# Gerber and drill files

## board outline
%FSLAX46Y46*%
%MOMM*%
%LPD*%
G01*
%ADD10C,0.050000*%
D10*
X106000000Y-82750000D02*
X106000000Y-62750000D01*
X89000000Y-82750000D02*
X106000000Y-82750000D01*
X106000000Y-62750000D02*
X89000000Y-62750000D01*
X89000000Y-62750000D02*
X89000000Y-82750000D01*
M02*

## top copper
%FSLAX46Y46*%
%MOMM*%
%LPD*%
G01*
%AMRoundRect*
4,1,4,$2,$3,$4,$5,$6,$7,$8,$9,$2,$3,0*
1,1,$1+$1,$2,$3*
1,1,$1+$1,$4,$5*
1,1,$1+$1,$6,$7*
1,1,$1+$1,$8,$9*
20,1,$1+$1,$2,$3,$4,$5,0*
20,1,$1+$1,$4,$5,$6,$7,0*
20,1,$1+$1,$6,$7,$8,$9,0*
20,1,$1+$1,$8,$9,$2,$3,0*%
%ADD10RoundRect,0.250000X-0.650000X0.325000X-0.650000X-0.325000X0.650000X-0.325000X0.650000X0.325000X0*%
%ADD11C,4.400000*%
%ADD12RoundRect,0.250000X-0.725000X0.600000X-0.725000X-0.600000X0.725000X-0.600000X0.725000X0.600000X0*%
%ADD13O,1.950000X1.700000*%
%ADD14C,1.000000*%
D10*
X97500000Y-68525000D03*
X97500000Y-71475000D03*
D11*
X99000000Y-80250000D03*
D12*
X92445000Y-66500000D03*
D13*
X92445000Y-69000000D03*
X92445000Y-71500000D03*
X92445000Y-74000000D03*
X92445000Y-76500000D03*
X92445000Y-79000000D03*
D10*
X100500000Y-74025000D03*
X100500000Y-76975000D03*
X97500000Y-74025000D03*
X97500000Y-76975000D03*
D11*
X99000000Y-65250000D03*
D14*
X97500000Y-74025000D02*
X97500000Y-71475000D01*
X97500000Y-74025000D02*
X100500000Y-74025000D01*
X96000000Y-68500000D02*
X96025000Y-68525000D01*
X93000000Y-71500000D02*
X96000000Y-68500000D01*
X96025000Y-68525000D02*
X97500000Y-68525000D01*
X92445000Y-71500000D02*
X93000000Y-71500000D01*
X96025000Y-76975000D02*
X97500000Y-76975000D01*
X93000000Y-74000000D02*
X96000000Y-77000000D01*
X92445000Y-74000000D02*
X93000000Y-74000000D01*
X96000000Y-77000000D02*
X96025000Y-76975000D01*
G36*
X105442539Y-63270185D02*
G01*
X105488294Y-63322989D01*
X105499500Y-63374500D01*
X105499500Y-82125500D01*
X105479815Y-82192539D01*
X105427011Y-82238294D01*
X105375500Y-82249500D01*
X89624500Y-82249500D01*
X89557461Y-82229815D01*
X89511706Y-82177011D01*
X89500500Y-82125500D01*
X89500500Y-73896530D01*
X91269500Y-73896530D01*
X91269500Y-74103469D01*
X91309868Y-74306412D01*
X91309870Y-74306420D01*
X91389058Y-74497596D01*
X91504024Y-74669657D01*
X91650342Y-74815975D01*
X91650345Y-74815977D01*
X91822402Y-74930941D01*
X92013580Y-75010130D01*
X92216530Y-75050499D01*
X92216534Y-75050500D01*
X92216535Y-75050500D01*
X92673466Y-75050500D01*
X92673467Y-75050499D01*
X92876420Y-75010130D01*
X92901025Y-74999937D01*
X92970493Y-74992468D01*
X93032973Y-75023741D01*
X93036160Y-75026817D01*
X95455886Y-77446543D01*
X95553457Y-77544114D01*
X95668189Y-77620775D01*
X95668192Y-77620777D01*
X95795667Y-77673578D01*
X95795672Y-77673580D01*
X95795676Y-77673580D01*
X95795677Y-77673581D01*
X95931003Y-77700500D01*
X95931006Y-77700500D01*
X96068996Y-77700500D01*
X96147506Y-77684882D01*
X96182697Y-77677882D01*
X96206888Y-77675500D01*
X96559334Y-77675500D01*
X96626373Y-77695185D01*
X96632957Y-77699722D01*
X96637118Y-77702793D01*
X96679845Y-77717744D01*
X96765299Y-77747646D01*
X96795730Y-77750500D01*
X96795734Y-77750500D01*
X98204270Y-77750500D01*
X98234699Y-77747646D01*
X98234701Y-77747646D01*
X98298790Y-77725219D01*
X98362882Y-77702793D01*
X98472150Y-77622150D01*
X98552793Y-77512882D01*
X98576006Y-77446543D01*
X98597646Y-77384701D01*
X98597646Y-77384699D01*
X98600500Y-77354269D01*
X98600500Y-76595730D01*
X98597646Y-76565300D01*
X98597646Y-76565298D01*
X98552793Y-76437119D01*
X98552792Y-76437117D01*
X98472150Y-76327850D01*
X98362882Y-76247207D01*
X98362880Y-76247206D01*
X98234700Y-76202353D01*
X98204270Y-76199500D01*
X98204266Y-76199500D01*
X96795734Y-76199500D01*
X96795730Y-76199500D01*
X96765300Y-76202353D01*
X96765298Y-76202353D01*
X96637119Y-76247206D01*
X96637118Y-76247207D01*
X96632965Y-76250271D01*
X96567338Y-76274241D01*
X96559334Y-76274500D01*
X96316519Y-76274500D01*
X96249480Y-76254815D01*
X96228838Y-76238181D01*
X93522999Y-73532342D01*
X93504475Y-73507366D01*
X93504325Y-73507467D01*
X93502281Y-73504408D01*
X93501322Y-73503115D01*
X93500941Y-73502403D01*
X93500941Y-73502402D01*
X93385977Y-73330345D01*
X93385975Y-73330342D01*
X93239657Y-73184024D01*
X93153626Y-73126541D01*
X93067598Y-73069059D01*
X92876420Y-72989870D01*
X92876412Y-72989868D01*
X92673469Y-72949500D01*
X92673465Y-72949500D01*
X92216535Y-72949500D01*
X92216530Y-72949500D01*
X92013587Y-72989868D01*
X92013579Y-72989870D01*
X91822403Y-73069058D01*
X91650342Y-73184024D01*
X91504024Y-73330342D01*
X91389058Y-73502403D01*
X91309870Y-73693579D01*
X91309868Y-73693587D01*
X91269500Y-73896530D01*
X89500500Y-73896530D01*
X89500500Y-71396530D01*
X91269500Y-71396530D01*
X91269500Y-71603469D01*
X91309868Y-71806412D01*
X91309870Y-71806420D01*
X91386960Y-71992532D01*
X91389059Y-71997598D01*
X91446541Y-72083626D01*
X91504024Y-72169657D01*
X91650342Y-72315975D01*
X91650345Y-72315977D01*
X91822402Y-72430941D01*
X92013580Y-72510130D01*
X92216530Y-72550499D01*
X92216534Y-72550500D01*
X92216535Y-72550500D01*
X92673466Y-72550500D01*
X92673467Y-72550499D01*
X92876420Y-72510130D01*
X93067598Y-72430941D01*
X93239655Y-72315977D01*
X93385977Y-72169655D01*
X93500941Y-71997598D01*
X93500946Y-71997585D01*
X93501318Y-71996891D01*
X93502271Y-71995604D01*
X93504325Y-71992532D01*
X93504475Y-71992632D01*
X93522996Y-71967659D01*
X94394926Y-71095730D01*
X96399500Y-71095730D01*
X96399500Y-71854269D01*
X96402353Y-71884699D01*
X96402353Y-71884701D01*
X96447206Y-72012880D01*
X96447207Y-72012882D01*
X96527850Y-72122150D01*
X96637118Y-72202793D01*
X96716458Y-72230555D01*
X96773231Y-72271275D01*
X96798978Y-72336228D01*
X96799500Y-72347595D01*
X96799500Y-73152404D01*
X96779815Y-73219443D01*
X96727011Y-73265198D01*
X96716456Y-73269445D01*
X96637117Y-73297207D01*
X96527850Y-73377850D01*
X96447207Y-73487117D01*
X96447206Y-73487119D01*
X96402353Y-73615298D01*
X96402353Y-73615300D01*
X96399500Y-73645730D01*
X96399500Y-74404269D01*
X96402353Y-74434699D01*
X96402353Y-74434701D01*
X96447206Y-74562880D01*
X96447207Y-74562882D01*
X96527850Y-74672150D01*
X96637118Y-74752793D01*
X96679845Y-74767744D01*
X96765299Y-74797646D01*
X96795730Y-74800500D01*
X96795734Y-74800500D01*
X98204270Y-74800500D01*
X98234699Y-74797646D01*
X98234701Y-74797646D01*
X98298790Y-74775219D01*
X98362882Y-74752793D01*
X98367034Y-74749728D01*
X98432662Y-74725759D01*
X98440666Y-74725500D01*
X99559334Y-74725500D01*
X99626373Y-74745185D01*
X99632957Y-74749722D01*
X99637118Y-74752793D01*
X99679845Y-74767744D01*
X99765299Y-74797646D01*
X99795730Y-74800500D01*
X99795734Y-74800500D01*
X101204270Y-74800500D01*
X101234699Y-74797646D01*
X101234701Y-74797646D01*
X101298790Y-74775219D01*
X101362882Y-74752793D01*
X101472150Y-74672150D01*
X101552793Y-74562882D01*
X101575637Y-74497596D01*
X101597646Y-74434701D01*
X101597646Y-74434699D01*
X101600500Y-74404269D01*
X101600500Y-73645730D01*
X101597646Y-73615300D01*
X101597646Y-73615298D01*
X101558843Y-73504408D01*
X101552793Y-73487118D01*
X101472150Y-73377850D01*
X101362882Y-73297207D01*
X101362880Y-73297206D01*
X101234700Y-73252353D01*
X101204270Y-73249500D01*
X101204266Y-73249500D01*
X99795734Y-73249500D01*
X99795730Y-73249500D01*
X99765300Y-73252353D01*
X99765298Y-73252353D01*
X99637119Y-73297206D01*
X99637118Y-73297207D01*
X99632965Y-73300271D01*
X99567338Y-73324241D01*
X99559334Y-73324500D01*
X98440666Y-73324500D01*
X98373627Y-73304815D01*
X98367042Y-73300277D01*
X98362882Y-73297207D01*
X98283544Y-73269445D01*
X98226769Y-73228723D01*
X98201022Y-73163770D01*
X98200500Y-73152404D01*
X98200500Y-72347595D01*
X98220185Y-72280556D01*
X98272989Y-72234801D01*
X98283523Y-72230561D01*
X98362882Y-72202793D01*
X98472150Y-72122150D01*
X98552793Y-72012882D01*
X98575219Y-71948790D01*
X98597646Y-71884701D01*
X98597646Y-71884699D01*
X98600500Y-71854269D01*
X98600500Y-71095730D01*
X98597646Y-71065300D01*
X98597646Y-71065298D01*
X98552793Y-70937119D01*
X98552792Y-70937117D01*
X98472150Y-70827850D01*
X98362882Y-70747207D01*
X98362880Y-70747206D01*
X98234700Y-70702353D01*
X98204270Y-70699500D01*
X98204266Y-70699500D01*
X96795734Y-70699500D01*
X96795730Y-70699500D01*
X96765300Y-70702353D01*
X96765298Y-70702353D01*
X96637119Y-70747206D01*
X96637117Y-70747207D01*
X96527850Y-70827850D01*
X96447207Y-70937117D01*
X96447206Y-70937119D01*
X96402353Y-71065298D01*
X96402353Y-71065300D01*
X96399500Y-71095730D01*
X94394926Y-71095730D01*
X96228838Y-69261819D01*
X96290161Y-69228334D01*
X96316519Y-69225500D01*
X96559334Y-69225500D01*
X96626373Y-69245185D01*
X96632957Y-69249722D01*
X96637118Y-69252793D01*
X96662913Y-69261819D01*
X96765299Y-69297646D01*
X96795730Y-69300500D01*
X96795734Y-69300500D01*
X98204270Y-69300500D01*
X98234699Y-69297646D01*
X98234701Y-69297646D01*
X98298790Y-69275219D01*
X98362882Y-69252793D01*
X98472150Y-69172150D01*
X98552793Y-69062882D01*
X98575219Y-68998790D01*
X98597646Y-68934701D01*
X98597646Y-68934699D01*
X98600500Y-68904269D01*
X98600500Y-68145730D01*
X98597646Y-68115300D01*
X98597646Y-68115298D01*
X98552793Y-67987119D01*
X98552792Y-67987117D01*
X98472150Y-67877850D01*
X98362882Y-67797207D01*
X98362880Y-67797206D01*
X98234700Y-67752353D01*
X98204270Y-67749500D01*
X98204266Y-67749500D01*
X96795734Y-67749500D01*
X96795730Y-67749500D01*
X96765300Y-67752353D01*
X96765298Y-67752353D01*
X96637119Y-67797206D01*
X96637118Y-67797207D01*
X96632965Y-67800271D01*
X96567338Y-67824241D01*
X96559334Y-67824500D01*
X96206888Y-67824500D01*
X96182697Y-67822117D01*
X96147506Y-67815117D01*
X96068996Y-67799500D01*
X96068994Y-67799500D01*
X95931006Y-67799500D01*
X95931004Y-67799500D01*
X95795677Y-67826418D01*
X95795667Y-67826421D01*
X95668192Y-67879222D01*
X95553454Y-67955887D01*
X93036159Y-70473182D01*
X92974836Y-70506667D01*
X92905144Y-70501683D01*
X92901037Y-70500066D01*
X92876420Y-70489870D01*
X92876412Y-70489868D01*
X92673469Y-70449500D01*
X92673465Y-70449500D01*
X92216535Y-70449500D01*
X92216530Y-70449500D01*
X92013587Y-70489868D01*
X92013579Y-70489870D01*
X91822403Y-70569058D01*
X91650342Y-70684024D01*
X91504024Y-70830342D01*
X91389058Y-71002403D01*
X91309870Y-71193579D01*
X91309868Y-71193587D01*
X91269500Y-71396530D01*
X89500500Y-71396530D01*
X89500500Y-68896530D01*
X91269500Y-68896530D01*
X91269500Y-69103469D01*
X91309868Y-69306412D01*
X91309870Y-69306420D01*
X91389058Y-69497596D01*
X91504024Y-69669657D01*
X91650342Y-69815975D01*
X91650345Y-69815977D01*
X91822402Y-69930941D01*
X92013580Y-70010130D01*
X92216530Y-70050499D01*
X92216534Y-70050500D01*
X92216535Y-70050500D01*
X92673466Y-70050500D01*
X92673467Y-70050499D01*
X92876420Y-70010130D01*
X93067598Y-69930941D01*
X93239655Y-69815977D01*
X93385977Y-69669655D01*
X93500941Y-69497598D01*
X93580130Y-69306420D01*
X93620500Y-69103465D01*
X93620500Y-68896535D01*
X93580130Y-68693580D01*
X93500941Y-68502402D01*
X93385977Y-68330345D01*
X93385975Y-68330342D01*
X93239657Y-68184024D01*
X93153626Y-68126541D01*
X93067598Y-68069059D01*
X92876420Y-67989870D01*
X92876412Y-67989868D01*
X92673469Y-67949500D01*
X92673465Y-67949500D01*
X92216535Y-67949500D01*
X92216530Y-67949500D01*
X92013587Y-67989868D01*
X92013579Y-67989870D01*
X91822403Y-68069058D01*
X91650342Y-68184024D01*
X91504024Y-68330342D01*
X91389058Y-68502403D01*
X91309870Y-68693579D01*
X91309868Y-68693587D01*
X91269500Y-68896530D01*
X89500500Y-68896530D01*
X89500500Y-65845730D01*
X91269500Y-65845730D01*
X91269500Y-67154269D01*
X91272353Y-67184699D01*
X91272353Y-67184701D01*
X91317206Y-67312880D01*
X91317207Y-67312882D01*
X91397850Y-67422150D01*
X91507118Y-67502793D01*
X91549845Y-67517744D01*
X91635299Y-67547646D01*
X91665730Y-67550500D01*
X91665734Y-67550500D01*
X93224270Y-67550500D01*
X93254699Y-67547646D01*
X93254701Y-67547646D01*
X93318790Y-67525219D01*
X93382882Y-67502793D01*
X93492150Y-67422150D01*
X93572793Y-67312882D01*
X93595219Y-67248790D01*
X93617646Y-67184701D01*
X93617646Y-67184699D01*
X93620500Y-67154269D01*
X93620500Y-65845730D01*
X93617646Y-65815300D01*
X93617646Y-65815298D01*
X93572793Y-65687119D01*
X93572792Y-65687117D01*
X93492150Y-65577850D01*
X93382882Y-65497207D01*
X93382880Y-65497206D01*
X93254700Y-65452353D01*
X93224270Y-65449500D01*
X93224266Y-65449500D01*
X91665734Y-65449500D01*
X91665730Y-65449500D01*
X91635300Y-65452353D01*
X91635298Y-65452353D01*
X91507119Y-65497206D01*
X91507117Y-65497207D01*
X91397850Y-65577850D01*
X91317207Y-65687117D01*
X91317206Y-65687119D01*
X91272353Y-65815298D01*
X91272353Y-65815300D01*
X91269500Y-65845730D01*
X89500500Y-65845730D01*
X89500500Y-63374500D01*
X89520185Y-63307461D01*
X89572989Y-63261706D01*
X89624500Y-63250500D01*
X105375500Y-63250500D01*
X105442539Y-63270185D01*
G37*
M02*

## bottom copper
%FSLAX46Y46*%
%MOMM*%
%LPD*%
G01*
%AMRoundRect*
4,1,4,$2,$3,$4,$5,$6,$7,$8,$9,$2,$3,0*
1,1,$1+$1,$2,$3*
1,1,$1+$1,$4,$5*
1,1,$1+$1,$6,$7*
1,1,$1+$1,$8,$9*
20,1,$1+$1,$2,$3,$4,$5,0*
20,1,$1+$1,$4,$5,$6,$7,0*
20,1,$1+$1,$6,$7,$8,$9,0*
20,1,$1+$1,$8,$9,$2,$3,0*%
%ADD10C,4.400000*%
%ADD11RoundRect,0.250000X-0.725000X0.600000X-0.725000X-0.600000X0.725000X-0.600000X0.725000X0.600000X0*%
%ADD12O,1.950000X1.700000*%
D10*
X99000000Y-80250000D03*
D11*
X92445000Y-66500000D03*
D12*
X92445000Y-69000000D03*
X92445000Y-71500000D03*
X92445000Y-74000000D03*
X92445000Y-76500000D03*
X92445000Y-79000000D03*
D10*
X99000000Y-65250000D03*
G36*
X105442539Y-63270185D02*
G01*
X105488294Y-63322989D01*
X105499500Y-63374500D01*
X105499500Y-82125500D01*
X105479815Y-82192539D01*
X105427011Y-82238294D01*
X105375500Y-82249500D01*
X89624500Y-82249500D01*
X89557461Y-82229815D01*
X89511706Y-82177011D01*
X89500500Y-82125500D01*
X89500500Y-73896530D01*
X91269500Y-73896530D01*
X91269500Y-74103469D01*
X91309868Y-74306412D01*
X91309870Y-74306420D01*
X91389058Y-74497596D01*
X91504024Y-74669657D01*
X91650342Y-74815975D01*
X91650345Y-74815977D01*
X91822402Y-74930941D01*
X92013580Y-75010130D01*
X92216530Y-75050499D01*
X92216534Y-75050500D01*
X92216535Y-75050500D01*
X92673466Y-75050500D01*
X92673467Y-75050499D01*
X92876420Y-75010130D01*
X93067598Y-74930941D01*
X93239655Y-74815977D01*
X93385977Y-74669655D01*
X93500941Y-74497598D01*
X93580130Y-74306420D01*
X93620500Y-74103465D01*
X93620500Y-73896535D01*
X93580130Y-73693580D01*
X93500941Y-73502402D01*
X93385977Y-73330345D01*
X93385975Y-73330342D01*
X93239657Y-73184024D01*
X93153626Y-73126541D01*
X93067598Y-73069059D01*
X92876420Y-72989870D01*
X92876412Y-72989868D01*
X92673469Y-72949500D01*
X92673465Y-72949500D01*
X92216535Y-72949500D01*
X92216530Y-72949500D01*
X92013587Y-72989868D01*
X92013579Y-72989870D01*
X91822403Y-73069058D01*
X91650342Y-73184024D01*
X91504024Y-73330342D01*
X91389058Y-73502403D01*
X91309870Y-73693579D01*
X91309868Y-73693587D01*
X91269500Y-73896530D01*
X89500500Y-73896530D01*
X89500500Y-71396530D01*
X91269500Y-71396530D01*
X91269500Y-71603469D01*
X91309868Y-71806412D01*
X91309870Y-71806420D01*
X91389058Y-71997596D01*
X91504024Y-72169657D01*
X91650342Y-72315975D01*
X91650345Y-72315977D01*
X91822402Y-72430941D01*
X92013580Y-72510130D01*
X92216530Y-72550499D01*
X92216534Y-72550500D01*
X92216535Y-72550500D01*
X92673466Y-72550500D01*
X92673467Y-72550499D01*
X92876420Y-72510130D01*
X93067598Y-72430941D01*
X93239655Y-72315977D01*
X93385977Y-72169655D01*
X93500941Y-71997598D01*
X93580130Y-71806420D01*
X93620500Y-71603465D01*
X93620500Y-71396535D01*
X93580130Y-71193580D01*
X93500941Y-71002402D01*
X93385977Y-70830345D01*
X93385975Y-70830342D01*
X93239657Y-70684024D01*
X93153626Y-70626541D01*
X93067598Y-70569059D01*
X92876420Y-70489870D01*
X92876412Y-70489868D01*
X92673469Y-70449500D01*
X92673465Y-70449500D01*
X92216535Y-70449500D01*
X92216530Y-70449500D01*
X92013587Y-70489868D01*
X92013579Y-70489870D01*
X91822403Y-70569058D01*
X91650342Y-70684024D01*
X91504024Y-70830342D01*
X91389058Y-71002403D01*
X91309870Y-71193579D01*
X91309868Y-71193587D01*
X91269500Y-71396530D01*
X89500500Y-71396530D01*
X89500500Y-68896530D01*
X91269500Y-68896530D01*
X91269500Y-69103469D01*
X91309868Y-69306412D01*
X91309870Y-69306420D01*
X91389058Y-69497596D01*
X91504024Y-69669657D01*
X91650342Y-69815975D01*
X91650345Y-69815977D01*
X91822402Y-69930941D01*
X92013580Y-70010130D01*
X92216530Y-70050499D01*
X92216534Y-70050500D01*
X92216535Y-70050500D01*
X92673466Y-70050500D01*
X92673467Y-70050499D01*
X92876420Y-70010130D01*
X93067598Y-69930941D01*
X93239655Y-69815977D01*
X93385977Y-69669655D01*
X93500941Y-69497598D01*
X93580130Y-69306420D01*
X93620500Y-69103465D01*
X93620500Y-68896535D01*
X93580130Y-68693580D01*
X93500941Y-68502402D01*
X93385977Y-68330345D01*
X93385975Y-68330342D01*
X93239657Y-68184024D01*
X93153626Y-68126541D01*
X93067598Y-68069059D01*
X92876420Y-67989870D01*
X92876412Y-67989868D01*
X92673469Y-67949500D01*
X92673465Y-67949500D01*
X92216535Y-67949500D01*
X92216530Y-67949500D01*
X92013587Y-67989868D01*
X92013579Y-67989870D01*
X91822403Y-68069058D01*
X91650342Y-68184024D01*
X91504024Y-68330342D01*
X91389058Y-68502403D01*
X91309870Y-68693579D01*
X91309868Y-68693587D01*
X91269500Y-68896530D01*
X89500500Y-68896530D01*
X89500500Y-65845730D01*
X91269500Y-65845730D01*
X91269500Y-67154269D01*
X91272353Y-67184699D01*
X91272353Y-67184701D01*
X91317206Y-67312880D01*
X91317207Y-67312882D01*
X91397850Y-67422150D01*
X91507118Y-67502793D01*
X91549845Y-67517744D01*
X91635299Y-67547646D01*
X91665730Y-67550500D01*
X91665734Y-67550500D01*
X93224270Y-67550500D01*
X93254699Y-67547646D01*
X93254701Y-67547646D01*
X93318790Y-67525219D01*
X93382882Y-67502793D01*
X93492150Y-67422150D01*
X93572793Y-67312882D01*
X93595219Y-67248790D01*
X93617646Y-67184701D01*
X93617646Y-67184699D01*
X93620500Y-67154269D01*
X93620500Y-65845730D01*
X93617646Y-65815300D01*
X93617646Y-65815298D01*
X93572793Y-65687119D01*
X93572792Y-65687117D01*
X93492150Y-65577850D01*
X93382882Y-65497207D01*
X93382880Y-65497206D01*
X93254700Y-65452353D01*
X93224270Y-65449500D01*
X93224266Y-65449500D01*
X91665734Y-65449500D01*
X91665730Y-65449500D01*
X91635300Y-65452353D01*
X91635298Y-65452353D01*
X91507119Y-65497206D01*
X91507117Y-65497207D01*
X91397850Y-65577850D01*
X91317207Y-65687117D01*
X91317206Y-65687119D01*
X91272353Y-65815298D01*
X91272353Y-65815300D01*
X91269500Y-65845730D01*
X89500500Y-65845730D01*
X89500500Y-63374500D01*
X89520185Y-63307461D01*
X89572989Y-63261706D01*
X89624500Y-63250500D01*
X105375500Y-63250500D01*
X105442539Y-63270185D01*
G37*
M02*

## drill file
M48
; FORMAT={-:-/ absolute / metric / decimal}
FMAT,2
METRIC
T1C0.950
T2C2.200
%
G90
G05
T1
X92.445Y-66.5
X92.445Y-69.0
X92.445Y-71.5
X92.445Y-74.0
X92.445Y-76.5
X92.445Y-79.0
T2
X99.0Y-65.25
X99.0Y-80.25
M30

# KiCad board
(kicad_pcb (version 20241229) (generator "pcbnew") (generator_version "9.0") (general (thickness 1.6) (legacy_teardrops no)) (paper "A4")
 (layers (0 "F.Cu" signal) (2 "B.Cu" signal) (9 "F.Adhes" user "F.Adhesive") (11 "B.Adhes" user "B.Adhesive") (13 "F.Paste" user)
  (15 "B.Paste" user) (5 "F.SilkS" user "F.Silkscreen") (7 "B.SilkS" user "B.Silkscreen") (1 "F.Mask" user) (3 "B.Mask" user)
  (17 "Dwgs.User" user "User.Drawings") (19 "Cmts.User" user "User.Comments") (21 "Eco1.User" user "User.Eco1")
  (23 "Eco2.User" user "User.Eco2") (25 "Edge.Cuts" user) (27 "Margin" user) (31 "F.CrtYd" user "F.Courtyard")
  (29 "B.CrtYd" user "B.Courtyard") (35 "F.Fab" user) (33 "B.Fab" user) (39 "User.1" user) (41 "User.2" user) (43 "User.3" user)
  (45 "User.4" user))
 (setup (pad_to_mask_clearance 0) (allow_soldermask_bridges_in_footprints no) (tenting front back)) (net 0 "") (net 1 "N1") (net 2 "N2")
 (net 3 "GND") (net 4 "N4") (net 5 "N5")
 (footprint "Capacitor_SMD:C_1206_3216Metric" (layer "F.Cu") (at 97.5 70 -90)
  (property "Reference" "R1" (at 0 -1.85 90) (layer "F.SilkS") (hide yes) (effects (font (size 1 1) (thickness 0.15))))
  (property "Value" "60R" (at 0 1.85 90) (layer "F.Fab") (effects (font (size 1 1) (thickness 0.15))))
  (pad "1" smd roundrect (at -1.475 0 270) (size 1.15 1.8) (layers "F.Cu" "F.Mask" "F.Paste") (roundrect_rratio 0.217391) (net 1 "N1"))
  (pad "2" smd roundrect (at 1.475 0 270) (size 1.15 1.8) (layers "F.Cu" "F.Mask" "F.Paste") (roundrect_rratio 0.217391) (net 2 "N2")))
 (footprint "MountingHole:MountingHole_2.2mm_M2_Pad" (layer "F.Cu") (at 99 80.25)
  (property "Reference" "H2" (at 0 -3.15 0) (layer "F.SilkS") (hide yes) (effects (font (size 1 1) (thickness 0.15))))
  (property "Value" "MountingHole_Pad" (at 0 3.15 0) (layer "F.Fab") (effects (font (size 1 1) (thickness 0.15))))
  (pad "1" thru_hole circle (at 0 0) (size 4.4 4.4) (drill 2.2) (layers "*.Cu" "*.Mask") (remove_unused_layers no) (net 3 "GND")
   (zone_connect 2)))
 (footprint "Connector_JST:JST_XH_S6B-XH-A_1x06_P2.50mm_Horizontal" (layer "F.Cu") (at 92.445 66.5 -90)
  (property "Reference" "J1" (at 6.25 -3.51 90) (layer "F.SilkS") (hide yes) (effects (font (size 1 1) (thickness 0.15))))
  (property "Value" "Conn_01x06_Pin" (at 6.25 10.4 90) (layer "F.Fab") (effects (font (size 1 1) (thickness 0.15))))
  (pad "1" thru_hole roundrect (at 0 0 270) (size 1.7 1.95) (drill 0.95) (layers "*.Cu" "*.Mask") (remove_unused_layers no)
   (roundrect_rratio 0.147059) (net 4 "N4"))
  (pad "2" thru_hole oval (at 2.5 0 270) (size 1.7 1.95) (drill 0.95) (layers "*.Cu" "*.Mask") (remove_unused_layers no) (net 4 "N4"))
  (pad "3" thru_hole oval (at 5 0 270) (size 1.7 1.95) (drill 0.95) (layers "*.Cu" "*.Mask") (remove_unused_layers no) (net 1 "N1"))
  (pad "4" thru_hole oval (at 7.5 0 270) (size 1.7 1.95) (drill 0.95) (layers "*.Cu" "*.Mask") (remove_unused_layers no) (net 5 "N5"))
  (pad "5" thru_hole oval (at 10 0 270) (size 1.7 1.95) (drill 0.95) (layers "*.Cu" "*.Mask") (remove_unused_layers no) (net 3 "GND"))
  (pad "6" thru_hole oval (at 12.5 0 270) (size 1.7 1.95) (drill 0.95) (layers "*.Cu" "*.Mask") (remove_unused_layers no) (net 3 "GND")))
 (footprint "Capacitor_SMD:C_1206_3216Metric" (layer "F.Cu") (at 100.5 75.5 -90)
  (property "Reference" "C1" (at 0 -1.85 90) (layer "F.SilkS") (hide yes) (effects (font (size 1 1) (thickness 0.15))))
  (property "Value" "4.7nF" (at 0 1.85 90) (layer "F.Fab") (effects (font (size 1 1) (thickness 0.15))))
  (pad "1" smd roundrect (at -1.475 0 270) (size 1.15 1.8) (layers "F.Cu" "F.Mask" "F.Paste") (roundrect_rratio 0.217391) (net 2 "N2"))
  (pad "2" smd roundrect (at 1.475 0 270) (size 1.15 1.8) (layers "F.Cu" "F.Mask" "F.Paste") (roundrect_rratio 0.217391) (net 3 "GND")))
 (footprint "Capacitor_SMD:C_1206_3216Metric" (layer "F.Cu") (at 97.5 75.5 -90)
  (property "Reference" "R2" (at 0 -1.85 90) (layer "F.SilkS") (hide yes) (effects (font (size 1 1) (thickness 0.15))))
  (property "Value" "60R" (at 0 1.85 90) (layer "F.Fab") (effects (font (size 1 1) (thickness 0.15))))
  (pad "1" smd roundrect (at -1.475 0 270) (size 1.15 1.8) (layers "F.Cu" "F.Mask" "F.Paste") (roundrect_rratio 0.217391) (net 2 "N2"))
  (pad "2" smd roundrect (at 1.475 0 270) (size 1.15 1.8) (layers "F.Cu" "F.Mask" "F.Paste") (roundrect_rratio 0.217391) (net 5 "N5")))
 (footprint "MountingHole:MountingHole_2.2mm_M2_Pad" (layer "F.Cu") (at 99 65.25)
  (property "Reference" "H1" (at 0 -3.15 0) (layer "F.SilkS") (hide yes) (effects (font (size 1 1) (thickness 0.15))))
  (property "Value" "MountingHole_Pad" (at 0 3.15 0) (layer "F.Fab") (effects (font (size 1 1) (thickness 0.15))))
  (pad "1" thru_hole circle (at 0 0) (size 4.4 4.4) (drill 2.2) (layers "*.Cu" "*.Mask") (remove_unused_layers no) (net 3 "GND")
   (zone_connect 2)))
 (gr_line (start 106 82.75) (end 106 62.75) (stroke (width 0.05) (type default)) (layer "Edge.Cuts"))
 (gr_line (start 89 82.75) (end 106 82.75) (stroke (width 0.05) (type default)) (layer "Edge.Cuts"))
 (gr_line (start 106 62.75) (end 89 62.75) (stroke (width 0.05) (type default)) (layer "Edge.Cuts"))
 (gr_line (start 89 62.75) (end 89 82.75) (stroke (width 0.05) (type default)) (layer "Edge.Cuts"))
 (segment (start 97.5 74.025) (end 97.5 71.475) (width 1) (layer "F.Cu") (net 2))
 (segment (start 97.5 74.025) (end 100.5 74.025) (width 1) (layer "F.Cu") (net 2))
 (segment (start 96 68.5) (end 96.025 68.525) (width 1) (layer "F.Cu") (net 1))
 (segment (start 93 71.5) (end 96 68.5) (width 1) (layer "F.Cu") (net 1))
 (segment (start 96.025 68.525) (end 97.5 68.525) (width 1) (layer "F.Cu") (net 1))
 (segment (start 92.445 71.5) (end 93 71.5) (width 1) (layer "F.Cu") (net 1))
 (segment (start 96.025 76.975) (end 97.5 76.975) (width 1) (layer "F.Cu") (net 5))
 (segment (start 93 74) (end 96 77) (width 1) (layer "F.Cu") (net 5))
 (segment (start 92.445 74) (end 93 74) (width 1) (layer "F.Cu") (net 5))
 (segment (start 96 77) (end 96.025 76.975) (width 1) (layer "F.Cu") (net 5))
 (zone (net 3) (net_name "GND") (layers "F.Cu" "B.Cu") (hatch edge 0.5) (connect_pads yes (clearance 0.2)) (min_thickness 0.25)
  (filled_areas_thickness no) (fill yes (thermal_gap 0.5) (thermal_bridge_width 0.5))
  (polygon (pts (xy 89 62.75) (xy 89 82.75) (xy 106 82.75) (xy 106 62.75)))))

